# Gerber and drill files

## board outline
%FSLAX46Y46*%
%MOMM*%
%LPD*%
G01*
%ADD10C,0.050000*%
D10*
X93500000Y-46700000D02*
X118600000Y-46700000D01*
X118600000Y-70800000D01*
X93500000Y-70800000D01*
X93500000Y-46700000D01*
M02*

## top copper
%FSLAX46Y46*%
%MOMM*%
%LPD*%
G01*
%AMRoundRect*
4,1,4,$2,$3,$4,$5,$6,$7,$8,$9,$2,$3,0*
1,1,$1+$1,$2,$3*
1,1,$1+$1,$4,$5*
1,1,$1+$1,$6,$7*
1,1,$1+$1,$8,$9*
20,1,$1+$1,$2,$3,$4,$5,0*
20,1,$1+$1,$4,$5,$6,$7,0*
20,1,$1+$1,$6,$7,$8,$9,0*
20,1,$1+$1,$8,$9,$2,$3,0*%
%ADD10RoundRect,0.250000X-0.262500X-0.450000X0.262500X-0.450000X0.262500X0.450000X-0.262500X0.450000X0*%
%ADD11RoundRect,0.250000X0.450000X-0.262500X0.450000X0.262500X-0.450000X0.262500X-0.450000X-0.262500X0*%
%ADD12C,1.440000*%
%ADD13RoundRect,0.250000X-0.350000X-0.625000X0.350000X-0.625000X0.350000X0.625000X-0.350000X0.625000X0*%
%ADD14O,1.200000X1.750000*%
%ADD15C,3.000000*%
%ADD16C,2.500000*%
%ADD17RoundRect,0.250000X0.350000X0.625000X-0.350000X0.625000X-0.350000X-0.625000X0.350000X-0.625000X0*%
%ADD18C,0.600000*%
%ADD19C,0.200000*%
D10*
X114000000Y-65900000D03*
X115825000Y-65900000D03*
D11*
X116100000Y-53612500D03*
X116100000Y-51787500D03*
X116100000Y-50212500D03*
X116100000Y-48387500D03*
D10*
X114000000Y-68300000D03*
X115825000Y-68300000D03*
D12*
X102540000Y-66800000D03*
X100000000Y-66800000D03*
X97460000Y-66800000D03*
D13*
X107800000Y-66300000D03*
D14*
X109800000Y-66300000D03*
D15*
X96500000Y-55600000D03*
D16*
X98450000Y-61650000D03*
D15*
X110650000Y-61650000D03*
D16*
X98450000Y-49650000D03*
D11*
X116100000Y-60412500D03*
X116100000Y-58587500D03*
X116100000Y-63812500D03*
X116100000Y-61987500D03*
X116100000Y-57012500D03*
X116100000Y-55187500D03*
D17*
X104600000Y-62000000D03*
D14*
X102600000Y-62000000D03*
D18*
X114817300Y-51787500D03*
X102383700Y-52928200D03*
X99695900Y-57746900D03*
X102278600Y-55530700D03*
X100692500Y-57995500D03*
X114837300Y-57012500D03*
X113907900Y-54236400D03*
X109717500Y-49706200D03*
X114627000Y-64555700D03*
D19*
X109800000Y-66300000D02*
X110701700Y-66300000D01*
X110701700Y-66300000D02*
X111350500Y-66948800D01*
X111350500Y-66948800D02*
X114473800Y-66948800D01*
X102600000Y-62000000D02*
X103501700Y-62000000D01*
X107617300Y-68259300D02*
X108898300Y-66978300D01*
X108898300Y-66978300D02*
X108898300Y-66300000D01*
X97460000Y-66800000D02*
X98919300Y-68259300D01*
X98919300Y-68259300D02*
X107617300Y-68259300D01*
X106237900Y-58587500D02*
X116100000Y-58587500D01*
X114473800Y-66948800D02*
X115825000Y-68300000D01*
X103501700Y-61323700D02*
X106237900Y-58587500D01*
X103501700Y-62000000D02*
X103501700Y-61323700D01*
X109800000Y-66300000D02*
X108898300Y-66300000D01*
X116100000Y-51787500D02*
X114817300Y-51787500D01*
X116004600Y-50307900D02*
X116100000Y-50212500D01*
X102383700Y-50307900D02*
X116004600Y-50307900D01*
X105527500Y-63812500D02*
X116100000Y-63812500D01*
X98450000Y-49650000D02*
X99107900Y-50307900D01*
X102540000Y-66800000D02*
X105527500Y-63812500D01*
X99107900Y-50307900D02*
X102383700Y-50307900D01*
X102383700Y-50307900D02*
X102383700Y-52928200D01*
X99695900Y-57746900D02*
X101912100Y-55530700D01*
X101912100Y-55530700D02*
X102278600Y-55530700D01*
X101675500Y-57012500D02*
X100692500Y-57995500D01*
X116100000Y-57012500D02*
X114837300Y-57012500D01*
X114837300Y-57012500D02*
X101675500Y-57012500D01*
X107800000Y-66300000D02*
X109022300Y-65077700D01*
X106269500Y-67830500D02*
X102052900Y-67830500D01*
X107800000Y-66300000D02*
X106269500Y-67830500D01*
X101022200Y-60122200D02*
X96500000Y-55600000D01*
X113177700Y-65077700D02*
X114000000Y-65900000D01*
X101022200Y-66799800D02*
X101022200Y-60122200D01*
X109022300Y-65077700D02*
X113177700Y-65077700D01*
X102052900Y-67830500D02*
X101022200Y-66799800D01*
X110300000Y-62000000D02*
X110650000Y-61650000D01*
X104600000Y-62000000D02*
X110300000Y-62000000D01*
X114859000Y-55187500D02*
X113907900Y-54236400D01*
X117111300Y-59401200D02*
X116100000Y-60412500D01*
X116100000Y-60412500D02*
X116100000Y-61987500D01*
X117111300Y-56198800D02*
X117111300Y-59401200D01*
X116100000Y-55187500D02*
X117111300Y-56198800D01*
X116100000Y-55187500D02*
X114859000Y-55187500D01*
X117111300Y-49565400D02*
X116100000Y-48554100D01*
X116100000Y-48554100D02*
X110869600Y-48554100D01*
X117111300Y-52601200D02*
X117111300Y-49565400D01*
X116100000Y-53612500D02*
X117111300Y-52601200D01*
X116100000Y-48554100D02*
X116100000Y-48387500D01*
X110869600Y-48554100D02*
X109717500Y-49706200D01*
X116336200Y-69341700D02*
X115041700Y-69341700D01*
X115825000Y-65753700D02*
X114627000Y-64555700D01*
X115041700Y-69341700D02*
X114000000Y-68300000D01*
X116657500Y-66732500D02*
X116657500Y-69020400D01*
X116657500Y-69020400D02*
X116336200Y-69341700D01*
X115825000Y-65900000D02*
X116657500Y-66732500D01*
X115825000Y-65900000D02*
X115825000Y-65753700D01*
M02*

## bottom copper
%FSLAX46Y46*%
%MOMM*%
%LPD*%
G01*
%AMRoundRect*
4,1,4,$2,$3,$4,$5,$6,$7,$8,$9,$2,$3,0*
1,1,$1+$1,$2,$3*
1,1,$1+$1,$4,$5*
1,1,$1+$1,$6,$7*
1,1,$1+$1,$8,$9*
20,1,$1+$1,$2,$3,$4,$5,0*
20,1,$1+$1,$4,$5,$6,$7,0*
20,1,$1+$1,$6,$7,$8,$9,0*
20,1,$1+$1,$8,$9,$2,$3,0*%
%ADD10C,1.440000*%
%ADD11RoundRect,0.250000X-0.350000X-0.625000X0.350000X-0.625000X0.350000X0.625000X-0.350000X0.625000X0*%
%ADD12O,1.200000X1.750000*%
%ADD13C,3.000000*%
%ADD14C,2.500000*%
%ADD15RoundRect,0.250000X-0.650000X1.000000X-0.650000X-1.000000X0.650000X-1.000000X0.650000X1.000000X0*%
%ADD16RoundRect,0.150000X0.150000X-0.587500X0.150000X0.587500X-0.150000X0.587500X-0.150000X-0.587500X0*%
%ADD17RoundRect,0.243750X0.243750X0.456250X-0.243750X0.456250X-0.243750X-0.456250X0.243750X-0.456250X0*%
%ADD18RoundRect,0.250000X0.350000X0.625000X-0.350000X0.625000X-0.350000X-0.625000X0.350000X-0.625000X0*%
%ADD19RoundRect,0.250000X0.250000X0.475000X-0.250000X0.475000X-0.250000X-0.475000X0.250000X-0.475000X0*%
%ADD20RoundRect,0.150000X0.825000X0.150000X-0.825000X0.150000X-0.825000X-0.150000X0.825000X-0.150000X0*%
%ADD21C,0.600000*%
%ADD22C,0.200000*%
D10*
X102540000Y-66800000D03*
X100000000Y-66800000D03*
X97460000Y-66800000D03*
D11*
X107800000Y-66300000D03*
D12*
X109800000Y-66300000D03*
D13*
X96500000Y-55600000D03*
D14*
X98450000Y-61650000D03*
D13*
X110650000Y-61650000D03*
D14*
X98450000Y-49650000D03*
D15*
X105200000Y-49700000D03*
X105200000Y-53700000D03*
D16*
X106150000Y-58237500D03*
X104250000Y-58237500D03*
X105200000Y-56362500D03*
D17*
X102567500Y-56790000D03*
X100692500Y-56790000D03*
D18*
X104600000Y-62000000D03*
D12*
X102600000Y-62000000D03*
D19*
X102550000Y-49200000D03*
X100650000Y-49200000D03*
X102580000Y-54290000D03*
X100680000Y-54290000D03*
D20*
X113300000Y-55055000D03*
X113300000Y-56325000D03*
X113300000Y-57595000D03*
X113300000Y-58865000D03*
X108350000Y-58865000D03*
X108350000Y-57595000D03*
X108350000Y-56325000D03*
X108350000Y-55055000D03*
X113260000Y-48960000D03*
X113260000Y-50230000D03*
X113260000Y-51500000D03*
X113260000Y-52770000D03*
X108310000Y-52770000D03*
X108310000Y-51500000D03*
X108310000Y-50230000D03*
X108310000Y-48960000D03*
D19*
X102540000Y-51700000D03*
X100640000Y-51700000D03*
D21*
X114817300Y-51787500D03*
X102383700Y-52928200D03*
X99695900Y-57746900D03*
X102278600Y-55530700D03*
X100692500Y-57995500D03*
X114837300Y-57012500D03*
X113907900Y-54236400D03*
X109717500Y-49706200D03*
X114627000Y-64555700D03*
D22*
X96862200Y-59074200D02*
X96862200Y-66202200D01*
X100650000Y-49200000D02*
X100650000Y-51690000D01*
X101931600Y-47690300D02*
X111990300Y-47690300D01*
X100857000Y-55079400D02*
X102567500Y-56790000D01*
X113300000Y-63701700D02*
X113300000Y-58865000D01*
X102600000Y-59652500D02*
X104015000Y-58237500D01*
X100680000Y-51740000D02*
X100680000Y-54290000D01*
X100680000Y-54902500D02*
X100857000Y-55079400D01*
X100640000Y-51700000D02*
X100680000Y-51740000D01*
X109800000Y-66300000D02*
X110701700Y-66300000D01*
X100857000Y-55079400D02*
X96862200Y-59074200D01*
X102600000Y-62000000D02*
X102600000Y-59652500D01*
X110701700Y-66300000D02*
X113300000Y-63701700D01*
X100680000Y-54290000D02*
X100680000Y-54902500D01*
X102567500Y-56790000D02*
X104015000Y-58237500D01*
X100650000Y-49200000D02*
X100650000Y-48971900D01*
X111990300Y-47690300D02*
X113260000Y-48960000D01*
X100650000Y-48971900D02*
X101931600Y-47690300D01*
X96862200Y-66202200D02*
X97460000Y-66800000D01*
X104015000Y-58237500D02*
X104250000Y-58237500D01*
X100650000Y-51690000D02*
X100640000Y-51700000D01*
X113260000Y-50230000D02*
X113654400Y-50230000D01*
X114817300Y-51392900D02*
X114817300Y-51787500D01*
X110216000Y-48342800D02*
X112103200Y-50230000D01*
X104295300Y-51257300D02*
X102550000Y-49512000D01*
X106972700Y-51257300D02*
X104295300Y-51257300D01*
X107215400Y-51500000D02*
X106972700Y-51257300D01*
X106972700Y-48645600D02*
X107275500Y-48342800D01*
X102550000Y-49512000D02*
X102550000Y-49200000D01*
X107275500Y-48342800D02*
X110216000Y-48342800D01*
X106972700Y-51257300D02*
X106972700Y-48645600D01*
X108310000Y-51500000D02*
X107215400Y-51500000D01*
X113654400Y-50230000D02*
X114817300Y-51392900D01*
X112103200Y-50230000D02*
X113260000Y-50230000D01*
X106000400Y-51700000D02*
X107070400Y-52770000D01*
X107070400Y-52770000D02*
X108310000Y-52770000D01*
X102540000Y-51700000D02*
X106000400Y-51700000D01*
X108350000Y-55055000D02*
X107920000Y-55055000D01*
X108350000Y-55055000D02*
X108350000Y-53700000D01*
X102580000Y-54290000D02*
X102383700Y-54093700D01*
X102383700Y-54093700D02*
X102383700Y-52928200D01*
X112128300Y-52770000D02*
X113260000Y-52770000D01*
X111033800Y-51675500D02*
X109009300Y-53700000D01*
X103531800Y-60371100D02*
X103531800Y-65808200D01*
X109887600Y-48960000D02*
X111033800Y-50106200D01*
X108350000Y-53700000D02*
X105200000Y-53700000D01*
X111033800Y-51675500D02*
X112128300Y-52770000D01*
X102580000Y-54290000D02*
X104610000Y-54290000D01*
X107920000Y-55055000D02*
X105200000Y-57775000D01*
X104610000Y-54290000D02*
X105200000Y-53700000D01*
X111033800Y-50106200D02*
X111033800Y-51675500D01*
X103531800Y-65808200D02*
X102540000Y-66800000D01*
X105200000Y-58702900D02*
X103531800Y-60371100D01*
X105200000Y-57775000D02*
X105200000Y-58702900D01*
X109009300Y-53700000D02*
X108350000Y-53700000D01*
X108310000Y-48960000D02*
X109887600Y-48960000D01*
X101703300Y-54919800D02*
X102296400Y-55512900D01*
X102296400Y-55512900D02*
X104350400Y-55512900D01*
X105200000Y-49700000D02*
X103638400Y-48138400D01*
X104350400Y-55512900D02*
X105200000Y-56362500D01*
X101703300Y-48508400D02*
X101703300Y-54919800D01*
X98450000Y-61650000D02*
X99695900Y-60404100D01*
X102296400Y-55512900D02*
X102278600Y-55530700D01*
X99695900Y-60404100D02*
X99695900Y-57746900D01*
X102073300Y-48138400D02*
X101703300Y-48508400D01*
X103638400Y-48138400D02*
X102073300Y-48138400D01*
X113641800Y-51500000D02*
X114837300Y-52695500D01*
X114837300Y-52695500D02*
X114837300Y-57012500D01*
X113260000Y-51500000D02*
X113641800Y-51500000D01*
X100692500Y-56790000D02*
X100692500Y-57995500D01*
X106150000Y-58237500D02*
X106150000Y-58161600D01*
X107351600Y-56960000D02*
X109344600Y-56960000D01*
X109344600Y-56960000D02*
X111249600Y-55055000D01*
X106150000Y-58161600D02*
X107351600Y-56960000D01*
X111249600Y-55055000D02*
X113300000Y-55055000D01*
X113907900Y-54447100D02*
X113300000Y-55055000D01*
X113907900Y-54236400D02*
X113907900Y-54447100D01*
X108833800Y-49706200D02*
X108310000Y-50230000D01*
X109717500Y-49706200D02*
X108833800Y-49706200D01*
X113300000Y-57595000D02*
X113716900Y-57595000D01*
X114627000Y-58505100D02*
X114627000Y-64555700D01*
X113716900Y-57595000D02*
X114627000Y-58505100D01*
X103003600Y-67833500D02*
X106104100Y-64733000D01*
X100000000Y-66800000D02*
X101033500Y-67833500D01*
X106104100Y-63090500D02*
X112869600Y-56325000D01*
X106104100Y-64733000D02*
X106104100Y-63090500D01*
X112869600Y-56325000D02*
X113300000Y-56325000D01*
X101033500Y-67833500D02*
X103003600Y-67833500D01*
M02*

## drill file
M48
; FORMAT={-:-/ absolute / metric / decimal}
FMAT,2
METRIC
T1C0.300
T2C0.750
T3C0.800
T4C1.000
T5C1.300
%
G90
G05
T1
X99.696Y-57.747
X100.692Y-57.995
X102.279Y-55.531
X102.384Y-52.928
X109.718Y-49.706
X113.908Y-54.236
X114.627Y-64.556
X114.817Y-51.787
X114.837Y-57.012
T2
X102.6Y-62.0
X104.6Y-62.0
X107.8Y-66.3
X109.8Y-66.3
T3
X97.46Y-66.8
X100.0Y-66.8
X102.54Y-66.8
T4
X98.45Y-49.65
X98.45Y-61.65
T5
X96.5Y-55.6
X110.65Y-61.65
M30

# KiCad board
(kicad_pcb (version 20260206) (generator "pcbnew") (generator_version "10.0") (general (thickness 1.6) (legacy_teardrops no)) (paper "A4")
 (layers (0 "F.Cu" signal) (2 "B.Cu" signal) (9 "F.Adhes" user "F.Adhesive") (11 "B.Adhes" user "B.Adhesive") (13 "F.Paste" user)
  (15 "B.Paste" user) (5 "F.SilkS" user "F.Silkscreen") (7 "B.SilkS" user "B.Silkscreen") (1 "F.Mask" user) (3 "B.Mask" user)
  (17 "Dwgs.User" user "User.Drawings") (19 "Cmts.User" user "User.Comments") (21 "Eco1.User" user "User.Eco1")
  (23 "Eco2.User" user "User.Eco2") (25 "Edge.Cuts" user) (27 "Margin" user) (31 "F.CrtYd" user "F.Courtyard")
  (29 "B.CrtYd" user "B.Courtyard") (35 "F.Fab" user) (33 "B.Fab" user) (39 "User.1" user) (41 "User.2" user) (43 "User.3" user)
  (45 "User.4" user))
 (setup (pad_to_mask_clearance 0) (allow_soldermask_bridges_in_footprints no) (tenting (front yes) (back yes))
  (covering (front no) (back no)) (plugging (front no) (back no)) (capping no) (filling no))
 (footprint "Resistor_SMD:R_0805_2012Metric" (layer "F.Cu") (at 114.9125 65.9)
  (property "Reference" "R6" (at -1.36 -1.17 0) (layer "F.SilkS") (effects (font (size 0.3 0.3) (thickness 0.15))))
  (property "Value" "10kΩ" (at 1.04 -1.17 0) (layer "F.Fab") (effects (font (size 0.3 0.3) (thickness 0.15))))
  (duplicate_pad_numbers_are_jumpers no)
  (pad "1" smd roundrect (at -0.9125 0) (size 1.025 1.4) (layers "F.Cu" "F.Mask" "F.Paste") (roundrect_rratio 0.243902) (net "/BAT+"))
  (pad "2" smd roundrect (at 0.9125 0) (size 1.025 1.4) (layers "F.Cu" "F.Mask" "F.Paste") (roundrect_rratio 0.243902) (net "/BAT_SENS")))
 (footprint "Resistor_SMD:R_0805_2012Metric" (layer "F.Cu") (at 116.1 52.7 90)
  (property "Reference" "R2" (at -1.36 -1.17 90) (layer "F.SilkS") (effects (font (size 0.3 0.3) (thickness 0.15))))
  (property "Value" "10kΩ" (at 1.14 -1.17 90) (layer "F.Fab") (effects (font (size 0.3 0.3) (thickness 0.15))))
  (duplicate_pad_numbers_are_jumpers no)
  (pad "1" smd roundrect (at -0.9125 0 90) (size 1.025 1.4) (layers "F.Cu" "F.Mask" "F.Paste") (roundrect_rratio 0.243902) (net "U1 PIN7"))
  (pad "2" smd roundrect (at 0.9125 0 90) (size 1.025 1.4) (layers "F.Cu" "F.Mask" "F.Paste") (roundrect_rratio 0.243902) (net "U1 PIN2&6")))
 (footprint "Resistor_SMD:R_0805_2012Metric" (layer "F.Cu") (at 116.1 49.3 90)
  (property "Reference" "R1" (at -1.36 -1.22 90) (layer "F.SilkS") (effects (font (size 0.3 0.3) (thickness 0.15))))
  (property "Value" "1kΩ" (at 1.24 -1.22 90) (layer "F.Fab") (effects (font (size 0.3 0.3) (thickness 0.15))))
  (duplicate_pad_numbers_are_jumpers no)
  (pad "1" smd roundrect (at -0.9125 0 90) (size 1.025 1.4) (layers "F.Cu" "F.Mask" "F.Paste") (roundrect_rratio 0.243902) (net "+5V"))
  (pad "2" smd roundrect (at 0.9125 0 90) (size 1.025 1.4) (layers "F.Cu" "F.Mask" "F.Paste") (roundrect_rratio 0.243902) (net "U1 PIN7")))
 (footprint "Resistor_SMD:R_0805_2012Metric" (layer "F.Cu") (at 114.9125 68.3)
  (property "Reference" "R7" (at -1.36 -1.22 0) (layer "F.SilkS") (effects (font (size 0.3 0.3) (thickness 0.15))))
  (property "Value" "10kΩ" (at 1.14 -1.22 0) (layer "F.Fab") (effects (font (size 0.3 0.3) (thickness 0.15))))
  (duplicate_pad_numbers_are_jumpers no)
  (pad "1" smd roundrect (at -0.9125 0) (size 1.025 1.4) (layers "F.Cu" "F.Mask" "F.Paste") (roundrect_rratio 0.243902) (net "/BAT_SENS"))
  (pad "2" smd roundrect (at 0.9125 0) (size 1.025 1.4) (layers "F.Cu" "F.Mask" "F.Paste") (roundrect_rratio 0.243902) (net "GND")))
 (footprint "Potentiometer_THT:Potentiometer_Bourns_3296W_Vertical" (layer "F.Cu") (at 102.54 66.8)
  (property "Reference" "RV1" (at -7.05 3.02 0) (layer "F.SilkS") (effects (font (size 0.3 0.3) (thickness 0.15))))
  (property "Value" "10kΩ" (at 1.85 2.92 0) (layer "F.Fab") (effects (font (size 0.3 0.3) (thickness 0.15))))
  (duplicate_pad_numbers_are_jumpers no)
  (pad "1" thru_hole circle (at 0 0) (size 1.44 1.44) (drill 0.8) (layers "*.Cu" "*.Mask") (remove_unused_layers no) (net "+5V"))
  (pad "2" thru_hole circle (at -2.54 0) (size 1.44 1.44) (drill 0.8) (layers "*.Cu" "*.Mask") (remove_unused_layers no) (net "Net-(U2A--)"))
  (pad "3" thru_hole circle (at -5.08 0) (size 1.44 1.44) (drill 0.8) (layers "*.Cu" "*.Mask") (remove_unused_layers no) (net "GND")))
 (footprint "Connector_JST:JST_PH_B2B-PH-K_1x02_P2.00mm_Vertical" (layer "F.Cu") (at 107.8 66.3)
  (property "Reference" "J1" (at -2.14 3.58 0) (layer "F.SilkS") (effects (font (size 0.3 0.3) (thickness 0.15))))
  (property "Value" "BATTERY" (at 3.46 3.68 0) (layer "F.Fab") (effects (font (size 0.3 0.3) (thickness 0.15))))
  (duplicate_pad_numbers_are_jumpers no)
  (pad "1" thru_hole roundrect (at 0 0) (size 1.2 1.75) (drill 0.75) (layers "*.Cu" "*.Mask") (remove_unused_layers no)
   (roundrect_rratio 0.208333) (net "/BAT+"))
  (pad "2" thru_hole oval (at 2 0) (size 1.2 1.75) (drill 0.75) (layers "*.Cu" "*.Mask") (remove_unused_layers no) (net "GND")))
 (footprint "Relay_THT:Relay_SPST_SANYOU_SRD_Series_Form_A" (layer "F.Cu") (at 96.5 55.6)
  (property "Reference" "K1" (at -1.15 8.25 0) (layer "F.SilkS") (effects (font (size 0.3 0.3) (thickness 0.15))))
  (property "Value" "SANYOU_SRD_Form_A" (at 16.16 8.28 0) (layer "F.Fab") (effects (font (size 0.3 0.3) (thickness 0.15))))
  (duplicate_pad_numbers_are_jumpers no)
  (pad "1" thru_hole circle (at 0 0 90) (size 3 3) (drill 1.3) (layers "*.Cu" "*.Mask") (remove_unused_layers no) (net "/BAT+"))
  (pad "2" thru_hole circle (at 1.95 6.05 90) (size 2.5 2.5) (drill 1) (layers "*.Cu" "*.Mask") (remove_unused_layers no) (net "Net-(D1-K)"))
  (pad "3" thru_hole circle (at 14.15 6.05 90) (size 3 3) (drill 1.3) (layers "*.Cu" "*.Mask") (remove_unused_layers no)
   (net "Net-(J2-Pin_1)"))
  (pad "5" thru_hole circle (at 1.95 -5.95 90) (size 2.5 2.5) (drill 1) (layers "*.Cu" "*.Mask") (remove_unused_layers no) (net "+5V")))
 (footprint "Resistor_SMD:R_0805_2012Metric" (layer "F.Cu") (at 116.1 59.5 90)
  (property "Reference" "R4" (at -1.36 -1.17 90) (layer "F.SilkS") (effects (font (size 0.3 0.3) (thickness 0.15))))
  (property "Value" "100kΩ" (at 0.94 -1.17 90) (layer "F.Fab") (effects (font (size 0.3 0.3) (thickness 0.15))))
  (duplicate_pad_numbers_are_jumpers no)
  (pad "1" smd roundrect (at -0.9125 0 90) (size 1.025 1.4) (layers "F.Cu" "F.Mask" "F.Paste") (roundrect_rratio 0.243902) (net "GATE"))
  (pad "2" smd roundrect (at 0.9125 0 90) (size 1.025 1.4) (layers "F.Cu" "F.Mask" "F.Paste") (roundrect_rratio 0.243902) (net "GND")))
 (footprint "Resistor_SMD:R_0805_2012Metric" (layer "F.Cu") (at 116.1 62.9 90)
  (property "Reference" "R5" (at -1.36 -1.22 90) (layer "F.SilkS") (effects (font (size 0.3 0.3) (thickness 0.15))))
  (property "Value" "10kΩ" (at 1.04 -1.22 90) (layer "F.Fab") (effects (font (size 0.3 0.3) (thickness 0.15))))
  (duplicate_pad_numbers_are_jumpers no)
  (pad "1" smd roundrect (at -0.9125 0 90) (size 1.025 1.4) (layers "F.Cu" "F.Mask" "F.Paste") (roundrect_rratio 0.243902) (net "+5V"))
  (pad "2" smd roundrect (at 0.9125 0 90) (size 1.025 1.4) (layers "F.Cu" "F.Mask" "F.Paste") (roundrect_rratio 0.243902) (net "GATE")))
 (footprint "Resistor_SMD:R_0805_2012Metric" (layer "F.Cu") (at 116.1 56.1 90)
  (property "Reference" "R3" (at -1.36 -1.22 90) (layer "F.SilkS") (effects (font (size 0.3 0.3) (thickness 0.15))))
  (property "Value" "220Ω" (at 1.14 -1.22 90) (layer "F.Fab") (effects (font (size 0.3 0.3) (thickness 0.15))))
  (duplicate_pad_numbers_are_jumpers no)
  (pad "1" smd roundrect (at -0.9125 0 90) (size 1.025 1.4) (layers "F.Cu" "F.Mask" "F.Paste") (roundrect_rratio 0.243902) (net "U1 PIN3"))
  (pad "2" smd roundrect (at 0.9125 0 90) (size 1.025 1.4) (layers "F.Cu" "F.Mask" "F.Paste") (roundrect_rratio 0.243902) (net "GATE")))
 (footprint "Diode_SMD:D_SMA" (layer "B.Cu") (at 105.2 51.7 -90)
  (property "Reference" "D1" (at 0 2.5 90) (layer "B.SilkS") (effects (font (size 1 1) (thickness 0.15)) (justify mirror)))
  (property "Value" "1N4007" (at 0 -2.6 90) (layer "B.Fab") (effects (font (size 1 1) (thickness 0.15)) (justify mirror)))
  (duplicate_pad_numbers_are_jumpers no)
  (pad "1" smd roundrect (at -2 0 270) (size 2.5 1.8) (layers "B.Cu" "B.Mask" "B.Paste") (roundrect_rratio 0.1388888889) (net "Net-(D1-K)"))
  (pad "2" smd roundrect (at 2 0 270) (size 2.5 1.8) (layers "B.Cu" "B.Mask" "B.Paste") (roundrect_rratio 0.1388888889) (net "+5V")))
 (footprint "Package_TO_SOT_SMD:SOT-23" (layer "B.Cu") (at 105.2 57.3 90)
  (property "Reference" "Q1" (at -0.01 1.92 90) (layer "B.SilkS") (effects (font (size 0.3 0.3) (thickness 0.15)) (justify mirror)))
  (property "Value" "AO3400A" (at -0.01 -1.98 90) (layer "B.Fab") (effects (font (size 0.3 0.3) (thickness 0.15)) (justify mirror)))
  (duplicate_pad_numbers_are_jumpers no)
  (pad "1" smd roundrect (at -0.9375 0.95 90) (size 1.475 0.6) (layers "B.Cu" "B.Mask" "B.Paste") (roundrect_rratio 0.25) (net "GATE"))
  (pad "2" smd roundrect (at -0.9375 -0.95 90) (size 1.475 0.6) (layers "B.Cu" "B.Mask" "B.Paste") (roundrect_rratio 0.25) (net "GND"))
  (pad "3" smd roundrect (at 0.9375 0 90) (size 1.475 0.6) (layers "B.Cu" "B.Mask" "B.Paste") (roundrect_rratio 0.25) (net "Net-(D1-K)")))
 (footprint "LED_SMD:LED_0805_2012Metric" (layer "B.Cu") (at 101.63 56.79 180)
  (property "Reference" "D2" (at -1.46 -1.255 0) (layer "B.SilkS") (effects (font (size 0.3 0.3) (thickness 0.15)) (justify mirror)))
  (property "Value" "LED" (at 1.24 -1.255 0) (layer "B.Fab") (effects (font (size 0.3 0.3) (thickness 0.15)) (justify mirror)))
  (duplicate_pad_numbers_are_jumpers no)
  (pad "1" smd roundrect (at -0.9375 0 180) (size 0.975 1.4) (layers "B.Cu" "B.Mask" "B.Paste") (roundrect_rratio 0.25) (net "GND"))
  (pad "2" smd roundrect (at 0.9375 0 180) (size 0.975 1.4) (layers "B.Cu" "B.Mask" "B.Paste") (roundrect_rratio 0.25) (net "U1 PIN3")))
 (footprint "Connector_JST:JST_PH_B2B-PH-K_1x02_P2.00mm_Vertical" (layer "B.Cu") (at 104.6 62 180)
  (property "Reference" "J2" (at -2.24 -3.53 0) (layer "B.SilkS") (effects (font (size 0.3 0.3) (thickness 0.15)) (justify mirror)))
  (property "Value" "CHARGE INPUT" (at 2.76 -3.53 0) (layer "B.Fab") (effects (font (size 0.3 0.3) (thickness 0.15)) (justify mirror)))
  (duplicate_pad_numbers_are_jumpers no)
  (pad "1" thru_hole roundrect (at 0 0 180) (size 1.2 1.75) (drill 0.75) (layers "*.Cu" "*.Mask") (remove_unused_layers no)
   (roundrect_rratio 0.208333) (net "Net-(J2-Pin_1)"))
  (pad "2" thru_hole oval (at 2 0 180) (size 1.2 1.75) (drill 0.75) (layers "*.Cu" "*.Mask") (remove_unused_layers no) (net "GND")))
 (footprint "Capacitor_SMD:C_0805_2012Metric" (layer "B.Cu") (at 101.6 49.2 180)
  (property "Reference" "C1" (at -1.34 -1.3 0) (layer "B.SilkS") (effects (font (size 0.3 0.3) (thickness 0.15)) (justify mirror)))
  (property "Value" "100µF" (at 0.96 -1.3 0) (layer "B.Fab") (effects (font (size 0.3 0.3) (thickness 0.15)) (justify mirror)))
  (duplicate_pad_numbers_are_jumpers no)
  (pad "1" smd roundrect (at -0.95 0 180) (size 1 1.45) (layers "B.Cu" "B.Mask" "B.Paste") (roundrect_rratio 0.25) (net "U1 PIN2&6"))
  (pad "2" smd roundrect (at 0.95 0 180) (size 1 1.45) (layers "B.Cu" "B.Mask" "B.Paste") (roundrect_rratio 0.25) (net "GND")))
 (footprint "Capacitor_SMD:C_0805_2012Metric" (layer "B.Cu") (at 101.63 54.29 180)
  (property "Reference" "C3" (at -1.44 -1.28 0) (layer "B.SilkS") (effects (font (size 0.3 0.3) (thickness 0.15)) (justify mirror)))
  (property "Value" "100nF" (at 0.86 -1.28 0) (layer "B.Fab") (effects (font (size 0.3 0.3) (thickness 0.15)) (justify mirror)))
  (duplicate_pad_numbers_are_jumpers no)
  (pad "1" smd roundrect (at -0.95 0 180) (size 1 1.45) (layers "B.Cu" "B.Mask" "B.Paste") (roundrect_rratio 0.25) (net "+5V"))
  (pad "2" smd roundrect (at 0.95 0 180) (size 1 1.45) (layers "B.Cu" "B.Mask" "B.Paste") (roundrect_rratio 0.25) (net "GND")))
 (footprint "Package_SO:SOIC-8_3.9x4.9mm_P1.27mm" (layer "B.Cu") (at 110.825 56.96 180)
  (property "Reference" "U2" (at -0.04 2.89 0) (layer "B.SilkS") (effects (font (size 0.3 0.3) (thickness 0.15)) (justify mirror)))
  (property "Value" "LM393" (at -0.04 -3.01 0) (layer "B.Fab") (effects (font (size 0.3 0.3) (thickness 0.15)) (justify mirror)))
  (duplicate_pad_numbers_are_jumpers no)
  (pad "1" smd roundrect (at -2.475 1.905 180) (size 1.95 0.6) (layers "B.Cu" "B.Mask" "B.Paste") (roundrect_rratio 0.25) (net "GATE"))
  (pad "2" smd roundrect (at -2.475 0.635 180) (size 1.95 0.6) (layers "B.Cu" "B.Mask" "B.Paste") (roundrect_rratio 0.25)
   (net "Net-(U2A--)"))
  (pad "3" smd roundrect (at -2.475 -0.635 180) (size 1.95 0.6) (layers "B.Cu" "B.Mask" "B.Paste") (roundrect_rratio 0.25) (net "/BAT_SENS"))
  (pad "4" smd roundrect (at -2.475 -1.905 180) (size 1.95 0.6) (layers "B.Cu" "B.Mask" "B.Paste") (roundrect_rratio 0.25) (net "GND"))
  (pad "5" smd roundrect (at 2.475 -1.905 180) (size 1.95 0.6) (layers "B.Cu" "B.Mask" "B.Paste") (roundrect_rratio 0.25)
   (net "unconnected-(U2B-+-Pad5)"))
  (pad "6" smd roundrect (at 2.475 -0.635 180) (size 1.95 0.6) (layers "B.Cu" "B.Mask" "B.Paste") (roundrect_rratio 0.25)
   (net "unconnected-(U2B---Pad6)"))
  (pad "7" smd roundrect (at 2.475 0.635 180) (size 1.95 0.6) (layers "B.Cu" "B.Mask" "B.Paste") (roundrect_rratio 0.25)
   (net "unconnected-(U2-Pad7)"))
  (pad "8" smd roundrect (at 2.475 1.905 180) (size 1.95 0.6) (layers "B.Cu" "B.Mask" "B.Paste") (roundrect_rratio 0.25) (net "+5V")))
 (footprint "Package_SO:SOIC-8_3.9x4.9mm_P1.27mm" (layer "B.Cu") (at 110.785 50.865 180)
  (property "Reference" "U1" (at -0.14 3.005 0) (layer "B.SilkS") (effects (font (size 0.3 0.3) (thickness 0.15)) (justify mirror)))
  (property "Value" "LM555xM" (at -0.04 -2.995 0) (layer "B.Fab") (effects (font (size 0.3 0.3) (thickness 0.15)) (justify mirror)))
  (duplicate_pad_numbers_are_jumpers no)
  (pad "1" smd roundrect (at -2.475 1.905 180) (size 1.95 0.6) (layers "B.Cu" "B.Mask" "B.Paste") (roundrect_rratio 0.25) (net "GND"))
  (pad "2" smd roundrect (at -2.475 0.635 180) (size 1.95 0.6) (layers "B.Cu" "B.Mask" "B.Paste") (roundrect_rratio 0.25) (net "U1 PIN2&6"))
  (pad "3" smd roundrect (at -2.475 -0.635 180) (size 1.95 0.6) (layers "B.Cu" "B.Mask" "B.Paste") (roundrect_rratio 0.25) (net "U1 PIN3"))
  (pad "4" smd roundrect (at -2.475 -1.905 180) (size 1.95 0.6) (layers "B.Cu" "B.Mask" "B.Paste") (roundrect_rratio 0.25) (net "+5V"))
  (pad "5" smd roundrect (at 2.475 -1.905 180) (size 1.95 0.6) (layers "B.Cu" "B.Mask" "B.Paste") (roundrect_rratio 0.25) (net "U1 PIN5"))
  (pad "6" smd roundrect (at 2.475 -0.635 180) (size 1.95 0.6) (layers "B.Cu" "B.Mask" "B.Paste") (roundrect_rratio 0.25) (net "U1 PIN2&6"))
  (pad "7" smd roundrect (at 2.475 0.635 180) (size 1.95 0.6) (layers "B.Cu" "B.Mask" "B.Paste") (roundrect_rratio 0.25) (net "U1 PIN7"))
  (pad "8" smd roundrect (at 2.475 1.905 180) (size 1.95 0.6) (layers "B.Cu" "B.Mask" "B.Paste") (roundrect_rratio 0.25) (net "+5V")))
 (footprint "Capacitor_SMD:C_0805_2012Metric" (layer "B.Cu") (at 101.59 51.7 180)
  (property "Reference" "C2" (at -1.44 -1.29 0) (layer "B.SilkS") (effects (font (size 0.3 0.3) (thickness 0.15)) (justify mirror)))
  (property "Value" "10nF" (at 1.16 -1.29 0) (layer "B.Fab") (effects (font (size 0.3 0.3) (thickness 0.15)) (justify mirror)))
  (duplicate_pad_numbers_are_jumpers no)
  (pad "1" smd roundrect (at -0.95 0 180) (size 1 1.45) (layers "B.Cu" "B.Mask" "B.Paste") (roundrect_rratio 0.25) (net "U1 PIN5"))
  (pad "2" smd roundrect (at 0.95 0 180) (size 1 1.45) (layers "B.Cu" "B.Mask" "B.Paste") (roundrect_rratio 0.25) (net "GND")))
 (gr_rect (start 93.5 46.7) (end 118.6 70.8) (stroke (width 0.05) (type default)) (fill no) (layer "Edge.Cuts"))
 (segment (start 109.8 66.3) (end 110.7017 66.3) (width 0.2) (layer "F.Cu") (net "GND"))
 (segment (start 110.7017 66.3) (end 111.3505 66.9488) (width 0.2) (layer "F.Cu") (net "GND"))
 (segment (start 111.3505 66.9488) (end 114.4738 66.9488) (width 0.2) (layer "F.Cu") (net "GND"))
 (segment (start 102.6 62) (end 103.5017 62) (width 0.2) (layer "F.Cu") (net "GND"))
 (segment (start 107.6173 68.2593) (end 108.8983 66.9783) (width 0.2) (layer "F.Cu") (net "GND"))
 (segment (start 108.8983 66.9783) (end 108.8983 66.3) (width 0.2) (layer "F.Cu") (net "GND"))
 (segment (start 97.46 66.8) (end 98.9193 68.2593) (width 0.2) (layer "F.Cu") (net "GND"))
 (segment (start 98.9193 68.2593) (end 107.6173 68.2593) (width 0.2) (layer "F.Cu") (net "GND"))
 (segment (start 106.2379 58.5875) (end 116.1 58.5875) (width 0.2) (layer "F.Cu") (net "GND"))
 (segment (start 114.4738 66.9488) (end 115.825 68.3) (width 0.2) (layer "F.Cu") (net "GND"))
 (segment (start 103.5017 61.3237) (end 106.2379 58.5875) (width 0.2) (layer "F.Cu") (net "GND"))
 (segment (start 103.5017 62) (end 103.5017 61.3237) (width 0.2) (layer "F.Cu") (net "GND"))
 (segment (start 109.8 66.3) (end 108.8983 66.3) (width 0.2) (layer "F.Cu") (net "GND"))
 (segment (start 96.8622 59.0742) (end 96.8622 66.2022) (width 0.2) (layer "B.Cu") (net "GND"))
 (segment (start 100.65 49.2) (end 100.65 51.69) (width 0.2) (layer "B.Cu") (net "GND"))
 (segment (start 101.9316 47.6903) (end 111.9903 47.6903) (width 0.2) (layer "B.Cu") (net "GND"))
 (segment (start 100.857 55.0794) (end 102.5675 56.79) (width 0.2) (layer "B.Cu") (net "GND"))
 (segment (start 113.3 63.7017) (end 113.3 58.865) (width 0.2) (layer "B.Cu") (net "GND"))
 (segment (start 102.6 59.6525) (end 104.015 58.2375) (width 0.2) (layer "B.Cu") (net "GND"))
 (segment (start 100.68 51.74) (end 100.68 54.29) (width 0.2) (layer "B.Cu") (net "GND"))
 (segment (start 100.68 54.9025) (end 100.857 55.0794) (width 0.2) (layer "B.Cu") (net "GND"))
 (segment (start 100.64 51.7) (end 100.68 51.74) (width 0.2) (layer "B.Cu") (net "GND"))
 (segment (start 109.8 66.3) (end 110.7017 66.3) (width 0.2) (layer "B.Cu") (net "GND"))
 (segment (start 100.857 55.0794) (end 96.8622 59.0742) (width 0.2) (layer "B.Cu") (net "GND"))
 (segment (start 102.6 62) (end 102.6 59.6525) (width 0.2) (layer "B.Cu") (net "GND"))
 (segment (start 110.7017 66.3) (end 113.3 63.7017) (width 0.2) (layer "B.Cu") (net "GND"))
 (segment (start 100.68 54.29) (end 100.68 54.9025) (width 0.2) (layer "B.Cu") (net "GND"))
 (segment (start 102.5675 56.79) (end 104.015 58.2375) (width 0.2) (layer "B.Cu") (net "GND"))
 (segment (start 100.65 49.2) (end 100.65 48.9719) (width 0.2) (layer "B.Cu") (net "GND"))
 (segment (start 111.9903 47.6903) (end 113.26 48.96) (width 0.2) (layer "B.Cu") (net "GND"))
 (segment (start 100.65 48.9719) (end 101.9316 47.6903) (width 0.2) (layer "B.Cu") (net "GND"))
 (segment (start 96.8622 66.2022) (end 97.46 66.8) (width 0.2) (layer "B.Cu") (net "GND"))
 (segment (start 104.015 58.2375) (end 104.25 58.2375) (width 0.2) (layer "B.Cu") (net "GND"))
 (segment (start 100.65 51.69) (end 100.64 51.7) (width 0.2) (layer "B.Cu") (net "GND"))
 (segment (start 116.1 51.7875) (end 114.8173 51.7875) (width 0.2) (layer "F.Cu") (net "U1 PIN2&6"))
 (via (at 114.8173 51.7875) (size 0.6) (drill 0.3) (layers "F.Cu" "B.Cu") (capping no) (covering (front no) (back no))
  (plugging (front no) (back no)) (filling no) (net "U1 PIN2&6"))
 (segment (start 113.26 50.23) (end 113.6544 50.23) (width 0.2) (layer "B.Cu") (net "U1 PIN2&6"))
 (segment (start 114.8173 51.3929) (end 114.8173 51.7875) (width 0.2) (layer "B.Cu") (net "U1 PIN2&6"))
 (segment (start 110.216 48.3428) (end 112.1032 50.23) (width 0.2) (layer "B.Cu") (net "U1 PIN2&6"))
 (segment (start 104.2953 51.2573) (end 102.55 49.512) (width 0.2) (layer "B.Cu") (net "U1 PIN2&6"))
 (segment (start 106.9727 51.2573) (end 104.2953 51.2573) (width 0.2) (layer "B.Cu") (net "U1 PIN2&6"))
 (segment (start 107.2154 51.5) (end 106.9727 51.2573) (width 0.2) (layer "B.Cu") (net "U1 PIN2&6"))
 (segment (start 106.9727 48.6456) (end 107.2755 48.3428) (width 0.2) (layer "B.Cu") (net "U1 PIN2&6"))
 (segment (start 102.55 49.512) (end 102.55 49.2) (width 0.2) (layer "B.Cu") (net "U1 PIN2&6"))
 (segment (start 107.2755 48.3428) (end 110.216 48.3428) (width 0.2) (layer "B.Cu") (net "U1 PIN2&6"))
 (segment (start 106.9727 51.2573) (end 106.9727 48.6456) (width 0.2) (layer "B.Cu") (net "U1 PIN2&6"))
 (segment (start 108.31 51.5) (end 107.2154 51.5) (width 0.2) (layer "B.Cu") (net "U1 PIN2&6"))
 (segment (start 113.6544 50.23) (end 114.8173 51.3929) (width 0.2) (layer "B.Cu") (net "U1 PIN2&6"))
 (segment (start 112.1032 50.23) (end 113.26 50.23) (width 0.2) (layer "B.Cu") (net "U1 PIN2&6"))
 (segment (start 106.0004 51.7) (end 107.0704 52.77) (width 0.2) (layer "B.Cu") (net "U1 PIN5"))
 (segment (start 107.0704 52.77) (end 108.31 52.77) (width 0.2) (layer "B.Cu") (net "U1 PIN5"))
 (segment (start 102.54 51.7) (end 106.0004 51.7) (width 0.2) (layer "B.Cu") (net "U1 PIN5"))
 (segment (start 116.0046 50.3079) (end 116.1 50.2125) (width 0.2) (layer "F.Cu") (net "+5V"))
 (segment (start 102.3837 50.3079) (end 116.0046 50.3079) (width 0.2) (layer "F.Cu") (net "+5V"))
 (segment (start 105.5275 63.8125) (end 116.1 63.8125) (width 0.2) (layer "F.Cu") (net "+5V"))
 (segment (start 98.45 49.65) (end 99.1079 50.3079) (width 0.2) (layer "F.Cu") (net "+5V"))
 (segment (start 102.54 66.8) (end 105.5275 63.8125) (width 0.2) (layer "F.Cu") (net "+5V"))
 (segment (start 99.1079 50.3079) (end 102.3837 50.3079) (width 0.2) (layer "F.Cu") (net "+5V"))
 (segment (start 102.3837 50.3079) (end 102.3837 52.9282) (width 0.2) (layer "F.Cu") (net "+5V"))
 (via (at 102.3837 52.9282) (size 0.6) (drill 0.3) (layers "F.Cu" "B.Cu") (capping no) (covering (front no) (back no))
  (plugging (front no) (back no)) (filling no) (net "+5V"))
 (segment (start 108.35 55.055) (end 107.92 55.055) (width 0.2) (layer "B.Cu") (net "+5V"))
 (segment (start 108.35 55.055) (end 108.35 53.7) (width 0.2) (layer "B.Cu") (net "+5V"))
 (segment (start 102.58 54.29) (end 102.3837 54.0937) (width 0.2) (layer "B.Cu") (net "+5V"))
 (segment (start 102.3837 54.0937) (end 102.3837 52.9282) (width 0.2) (layer "B.Cu") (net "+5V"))
 (segment (start 112.1283 52.77) (end 113.26 52.77) (width 0.2) (layer "B.Cu") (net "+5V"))
 (segment (start 111.0338 51.6755) (end 109.0093 53.7) (width 0.2) (layer "B.Cu") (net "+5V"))
 (segment (start 103.5318 60.3711) (end 103.5318 65.8082) (width 0.2) (layer "B.Cu") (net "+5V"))
 (segment (start 109.8876 48.96) (end 111.0338 50.1062) (width 0.2) (layer "B.Cu") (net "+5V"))
 (segment (start 108.35 53.7) (end 105.2 53.7) (width 0.2) (layer "B.Cu") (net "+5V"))
 (segment (start 111.0338 51.6755) (end 112.1283 52.77) (width 0.2) (layer "B.Cu") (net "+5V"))
 (segment (start 102.58 54.29) (end 104.61 54.29) (width 0.2) (layer "B.Cu") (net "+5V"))
 (segment (start 107.92 55.055) (end 105.2 57.775) (width 0.2) (layer "B.Cu") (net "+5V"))
 (segment (start 104.61 54.29) (end 105.2 53.7) (width 0.2) (layer "B.Cu") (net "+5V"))
 (segment (start 111.0338 50.1062) (end 111.0338 51.6755) (width 0.2) (layer "B.Cu") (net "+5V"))
 (segment (start 103.5318 65.8082) (end 102.54 66.8) (width 0.2) (layer "B.Cu") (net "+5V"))
 (segment (start 105.2 58.7029) (end 103.5318 60.3711) (width 0.2) (layer "B.Cu") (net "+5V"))
 (segment (start 105.2 57.775) (end 105.2 58.7029) (width 0.2) (layer "B.Cu") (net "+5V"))
 (segment (start 109.0093 53.7) (end 108.35 53.7) (width 0.2) (layer "B.Cu") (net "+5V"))
 (segment (start 108.31 48.96) (end 109.8876 48.96) (width 0.2) (layer "B.Cu") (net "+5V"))
 (segment (start 99.6959 57.7469) (end 101.9121 55.5307) (width 0.2) (layer "F.Cu") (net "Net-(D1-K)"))
 (segment (start 101.9121 55.5307) (end 102.2786 55.5307) (width 0.2) (layer "F.Cu") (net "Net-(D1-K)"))
 (via (at 99.6959 57.7469) (size 0.6) (drill 0.3) (layers "F.Cu" "B.Cu") (capping no) (covering (front no) (back no))
  (plugging (front no) (back no)) (filling no) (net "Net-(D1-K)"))
 (via (at 102.2786 55.5307) (size 0.6) (drill 0.3) (layers "F.Cu" "B.Cu") (capping no) (covering (front no) (back no))
  (plugging (front no) (back no)) (filling no) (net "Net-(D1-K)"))
 (segment (start 101.7033 54.9198) (end 102.2964 55.5129) (width 0.2) (layer "B.Cu") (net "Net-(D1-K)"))
 (segment (start 102.2964 55.5129) (end 104.3504 55.5129) (width 0.2) (layer "B.Cu") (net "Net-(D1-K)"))
 (segment (start 105.2 49.7) (end 103.6384 48.1384) (width 0.2) (layer "B.Cu") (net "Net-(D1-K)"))
 (segment (start 104.3504 55.5129) (end 105.2 56.3625) (width 0.2) (layer "B.Cu") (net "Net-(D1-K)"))
 (segment (start 101.7033 48.5084) (end 101.7033 54.9198) (width 0.2) (layer "B.Cu") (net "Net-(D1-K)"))
 (segment (start 98.45 61.65) (end 99.6959 60.4041) (width 0.2) (layer "B.Cu") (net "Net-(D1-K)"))
 (segment (start 102.2964 55.5129) (end 102.2786 55.5307) (width 0.2) (layer "B.Cu") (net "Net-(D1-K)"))
 (segment (start 99.6959 60.4041) (end 99.6959 57.7469) (width 0.2) (layer "B.Cu") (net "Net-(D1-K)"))
 (segment (start 102.0733 48.1384) (end 101.7033 48.5084) (width 0.2) (layer "B.Cu") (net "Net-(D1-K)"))
 (segment (start 103.6384 48.1384) (end 102.0733 48.1384) (width 0.2) (layer "B.Cu") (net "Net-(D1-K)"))
 (segment (start 101.6755 57.0125) (end 100.6925 57.9955) (width 0.2) (layer "F.Cu") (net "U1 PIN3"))
 (segment (start 116.1 57.0125) (end 114.8373 57.0125) (width 0.2) (layer "F.Cu") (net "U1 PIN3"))
 (segment (start 114.8373 57.0125) (end 101.6755 57.0125) (width 0.2) (layer "F.Cu") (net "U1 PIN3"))
 (via (at 100.6925 57.9955) (size 0.6) (drill 0.3) (layers "F.Cu" "B.Cu") (capping no) (covering (front no) (back no))
  (plugging (front no) (back no)) (filling no) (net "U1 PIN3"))
 (via (at 114.8373 57.0125) (size 0.6) (drill 0.3) (layers "F.Cu" "B.Cu") (capping no) (covering (front no) (back no))
  (plugging (front no) (back no)) (filling no) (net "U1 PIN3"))
 (segment (start 113.6418 51.5) (end 114.8373 52.6955) (width 0.2) (layer "B.Cu") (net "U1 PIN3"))
 (segment (start 114.8373 52.6955) (end 114.8373 57.0125) (width 0.2) (layer "B.Cu") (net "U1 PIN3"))
 (segment (start 113.26 51.5) (end 113.6418 51.5) (width 0.2) (layer "B.Cu") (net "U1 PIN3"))
 (segment (start 100.6925 56.79) (end 100.6925 57.9955) (width 0.2) (layer "B.Cu") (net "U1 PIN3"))
 (segment (start 107.8 66.3) (end 109.0223 65.0777) (width 0.2) (layer "F.Cu") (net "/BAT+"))
 (segment (start 106.2695 67.8305) (end 102.0529 67.8305) (width 0.2) (layer "F.Cu") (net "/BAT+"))
 (segment (start 107.8 66.3) (end 106.2695 67.8305) (width 0.2) (layer "F.Cu") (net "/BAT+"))
 (segment (start 101.0222 60.1222) (end 96.5 55.6) (width 0.2) (layer "F.Cu") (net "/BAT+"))
 (segment (start 113.1777 65.0777) (end 114 65.9) (width 0.2) (layer "F.Cu") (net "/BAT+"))
 (segment (start 101.0222 66.7998) (end 101.0222 60.1222) (width 0.2) (layer "F.Cu") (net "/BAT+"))
 (segment (start 109.0223 65.0777) (end 113.1777 65.0777) (width 0.2) (layer "F.Cu") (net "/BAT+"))
 (segment (start 102.0529 67.8305) (end 101.0222 66.7998) (width 0.2) (layer "F.Cu") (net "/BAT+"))
 (segment (start 110.3 62) (end 110.65 61.65) (width 0.2) (layer "F.Cu") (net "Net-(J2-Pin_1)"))
 (segment (start 104.6 62) (end 110.3 62) (width 0.2) (layer "F.Cu") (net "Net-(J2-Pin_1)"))
 (segment (start 114.859 55.1875) (end 113.9079 54.2364) (width 0.2) (layer "F.Cu") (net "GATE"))
 (segment (start 117.1113 59.4012) (end 116.1 60.4125) (width 0.2) (layer "F.Cu") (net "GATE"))
 (segment (start 116.1 60.4125) (end 116.1 61.9875) (width 0.2) (layer "F.Cu") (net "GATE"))
 (segment (start 117.1113 56.1988) (end 117.1113 59.4012) (width 0.2) (layer "F.Cu") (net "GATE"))
 (segment (start 116.1 55.1875) (end 117.1113 56.1988) (width 0.2) (layer "F.Cu") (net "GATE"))
 (segment (start 116.1 55.1875) (end 114.859 55.1875) (width 0.2) (layer "F.Cu") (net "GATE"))
 (via (at 113.9079 54.2364) (size 0.6) (drill 0.3) (layers "F.Cu" "B.Cu") (capping no) (covering (front no) (back no))
  (plugging (front no) (back no)) (filling no) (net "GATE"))
 (segment (start 106.15 58.2375) (end 106.15 58.1616) (width 0.2) (layer "B.Cu") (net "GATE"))
 (segment (start 107.3516 56.96) (end 109.3446 56.96) (width 0.2) (layer "B.Cu") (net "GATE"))
 (segment (start 109.3446 56.96) (end 111.2496 55.055) (width 0.2) (layer "B.Cu") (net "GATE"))
 (segment (start 106.15 58.1616) (end 107.3516 56.96) (width 0.2) (layer "B.Cu") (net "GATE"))
 (segment (start 111.2496 55.055) (end 113.3 55.055) (width 0.2) (layer "B.Cu") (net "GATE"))
 (segment (start 113.9079 54.4471) (end 113.3 55.055) (width 0.2) (layer "B.Cu") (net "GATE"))
 (segment (start 113.9079 54.2364) (end 113.9079 54.4471) (width 0.2) (layer "B.Cu") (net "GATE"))
 (segment (start 117.1113 49.5654) (end 116.1 48.5541) (width 0.2) (layer "F.Cu") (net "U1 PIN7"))
 (segment (start 116.1 48.5541) (end 110.8696 48.5541) (width 0.2) (layer "F.Cu") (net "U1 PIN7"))
 (segment (start 117.1113 52.6012) (end 117.1113 49.5654) (width 0.2) (layer "F.Cu") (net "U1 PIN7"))
 (segment (start 116.1 53.6125) (end 117.1113 52.6012) (width 0.2) (layer "F.Cu") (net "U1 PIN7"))
 (segment (start 116.1 48.5541) (end 116.1 48.3875) (width 0.2) (layer "F.Cu") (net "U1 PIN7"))
 (segment (start 110.8696 48.5541) (end 109.7175 49.7062) (width 0.2) (layer "F.Cu") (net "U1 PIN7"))
 (via (at 109.7175 49.7062) (size 0.6) (drill 0.3) (layers "F.Cu" "B.Cu") (capping no) (covering (front no) (back no))
  (plugging (front no) (back no)) (filling no) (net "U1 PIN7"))
 (segment (start 108.8338 49.7062) (end 108.31 50.23) (width 0.2) (layer "B.Cu") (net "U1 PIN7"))
 (segment (start 109.7175 49.7062) (end 108.8338 49.7062) (width 0.2) (layer "B.Cu") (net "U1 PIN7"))
 (segment (start 116.3362 69.3417) (end 115.0417 69.3417) (width 0.2) (layer "F.Cu") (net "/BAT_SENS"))
 (segment (start 115.825 65.7537) (end 114.627 64.5557) (width 0.2) (layer "F.Cu") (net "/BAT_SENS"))
 (segment (start 115.0417 69.3417) (end 114 68.3) (width 0.2) (layer "F.Cu") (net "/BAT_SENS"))
 (segment (start 116.6575 66.7325) (end 116.6575 69.0204) (width 0.2) (layer "F.Cu") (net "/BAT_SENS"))
 (segment (start 116.6575 69.0204) (end 116.3362 69.3417) (width 0.2) (layer "F.Cu") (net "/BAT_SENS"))
 (segment (start 115.825 65.9) (end 116.6575 66.7325) (width 0.2) (layer "F.Cu") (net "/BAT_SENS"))
 (segment (start 115.825 65.9) (end 115.825 65.7537) (width 0.2) (layer "F.Cu") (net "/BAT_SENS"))
 (via (at 114.627 64.5557) (size 0.6) (drill 0.3) (layers "F.Cu" "B.Cu") (capping no) (covering (front no) (back no))
  (plugging (front no) (back no)) (filling no) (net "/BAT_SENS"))
 (segment (start 113.3 57.595) (end 113.7169 57.595) (width 0.2) (layer "B.Cu") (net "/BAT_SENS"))
 (segment (start 114.627 58.5051) (end 114.627 64.5557) (width 0.2) (layer "B.Cu") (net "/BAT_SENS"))
 (segment (start 113.7169 57.595) (end 114.627 58.5051) (width 0.2) (layer "B.Cu") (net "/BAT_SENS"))
 (segment (start 103.0036 67.8335) (end 106.1041 64.733) (width 0.2) (layer "B.Cu") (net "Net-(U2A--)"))
 (segment (start 100 66.8) (end 101.0335 67.8335) (width 0.2) (layer "B.Cu") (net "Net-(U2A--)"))
 (segment (start 106.1041 63.0905) (end 112.8696 56.325) (width 0.2) (layer "B.Cu") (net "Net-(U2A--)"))
 (segment (start 106.1041 64.733) (end 106.1041 63.0905) (width 0.2) (layer "B.Cu") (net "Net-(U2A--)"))
 (segment (start 112.8696 56.325) (end 113.3 56.325) (width 0.2) (layer "B.Cu") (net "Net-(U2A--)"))
 (segment (start 101.0335 67.8335) (end 103.0036 67.8335) (width 0.2) (layer "B.Cu") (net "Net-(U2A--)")))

